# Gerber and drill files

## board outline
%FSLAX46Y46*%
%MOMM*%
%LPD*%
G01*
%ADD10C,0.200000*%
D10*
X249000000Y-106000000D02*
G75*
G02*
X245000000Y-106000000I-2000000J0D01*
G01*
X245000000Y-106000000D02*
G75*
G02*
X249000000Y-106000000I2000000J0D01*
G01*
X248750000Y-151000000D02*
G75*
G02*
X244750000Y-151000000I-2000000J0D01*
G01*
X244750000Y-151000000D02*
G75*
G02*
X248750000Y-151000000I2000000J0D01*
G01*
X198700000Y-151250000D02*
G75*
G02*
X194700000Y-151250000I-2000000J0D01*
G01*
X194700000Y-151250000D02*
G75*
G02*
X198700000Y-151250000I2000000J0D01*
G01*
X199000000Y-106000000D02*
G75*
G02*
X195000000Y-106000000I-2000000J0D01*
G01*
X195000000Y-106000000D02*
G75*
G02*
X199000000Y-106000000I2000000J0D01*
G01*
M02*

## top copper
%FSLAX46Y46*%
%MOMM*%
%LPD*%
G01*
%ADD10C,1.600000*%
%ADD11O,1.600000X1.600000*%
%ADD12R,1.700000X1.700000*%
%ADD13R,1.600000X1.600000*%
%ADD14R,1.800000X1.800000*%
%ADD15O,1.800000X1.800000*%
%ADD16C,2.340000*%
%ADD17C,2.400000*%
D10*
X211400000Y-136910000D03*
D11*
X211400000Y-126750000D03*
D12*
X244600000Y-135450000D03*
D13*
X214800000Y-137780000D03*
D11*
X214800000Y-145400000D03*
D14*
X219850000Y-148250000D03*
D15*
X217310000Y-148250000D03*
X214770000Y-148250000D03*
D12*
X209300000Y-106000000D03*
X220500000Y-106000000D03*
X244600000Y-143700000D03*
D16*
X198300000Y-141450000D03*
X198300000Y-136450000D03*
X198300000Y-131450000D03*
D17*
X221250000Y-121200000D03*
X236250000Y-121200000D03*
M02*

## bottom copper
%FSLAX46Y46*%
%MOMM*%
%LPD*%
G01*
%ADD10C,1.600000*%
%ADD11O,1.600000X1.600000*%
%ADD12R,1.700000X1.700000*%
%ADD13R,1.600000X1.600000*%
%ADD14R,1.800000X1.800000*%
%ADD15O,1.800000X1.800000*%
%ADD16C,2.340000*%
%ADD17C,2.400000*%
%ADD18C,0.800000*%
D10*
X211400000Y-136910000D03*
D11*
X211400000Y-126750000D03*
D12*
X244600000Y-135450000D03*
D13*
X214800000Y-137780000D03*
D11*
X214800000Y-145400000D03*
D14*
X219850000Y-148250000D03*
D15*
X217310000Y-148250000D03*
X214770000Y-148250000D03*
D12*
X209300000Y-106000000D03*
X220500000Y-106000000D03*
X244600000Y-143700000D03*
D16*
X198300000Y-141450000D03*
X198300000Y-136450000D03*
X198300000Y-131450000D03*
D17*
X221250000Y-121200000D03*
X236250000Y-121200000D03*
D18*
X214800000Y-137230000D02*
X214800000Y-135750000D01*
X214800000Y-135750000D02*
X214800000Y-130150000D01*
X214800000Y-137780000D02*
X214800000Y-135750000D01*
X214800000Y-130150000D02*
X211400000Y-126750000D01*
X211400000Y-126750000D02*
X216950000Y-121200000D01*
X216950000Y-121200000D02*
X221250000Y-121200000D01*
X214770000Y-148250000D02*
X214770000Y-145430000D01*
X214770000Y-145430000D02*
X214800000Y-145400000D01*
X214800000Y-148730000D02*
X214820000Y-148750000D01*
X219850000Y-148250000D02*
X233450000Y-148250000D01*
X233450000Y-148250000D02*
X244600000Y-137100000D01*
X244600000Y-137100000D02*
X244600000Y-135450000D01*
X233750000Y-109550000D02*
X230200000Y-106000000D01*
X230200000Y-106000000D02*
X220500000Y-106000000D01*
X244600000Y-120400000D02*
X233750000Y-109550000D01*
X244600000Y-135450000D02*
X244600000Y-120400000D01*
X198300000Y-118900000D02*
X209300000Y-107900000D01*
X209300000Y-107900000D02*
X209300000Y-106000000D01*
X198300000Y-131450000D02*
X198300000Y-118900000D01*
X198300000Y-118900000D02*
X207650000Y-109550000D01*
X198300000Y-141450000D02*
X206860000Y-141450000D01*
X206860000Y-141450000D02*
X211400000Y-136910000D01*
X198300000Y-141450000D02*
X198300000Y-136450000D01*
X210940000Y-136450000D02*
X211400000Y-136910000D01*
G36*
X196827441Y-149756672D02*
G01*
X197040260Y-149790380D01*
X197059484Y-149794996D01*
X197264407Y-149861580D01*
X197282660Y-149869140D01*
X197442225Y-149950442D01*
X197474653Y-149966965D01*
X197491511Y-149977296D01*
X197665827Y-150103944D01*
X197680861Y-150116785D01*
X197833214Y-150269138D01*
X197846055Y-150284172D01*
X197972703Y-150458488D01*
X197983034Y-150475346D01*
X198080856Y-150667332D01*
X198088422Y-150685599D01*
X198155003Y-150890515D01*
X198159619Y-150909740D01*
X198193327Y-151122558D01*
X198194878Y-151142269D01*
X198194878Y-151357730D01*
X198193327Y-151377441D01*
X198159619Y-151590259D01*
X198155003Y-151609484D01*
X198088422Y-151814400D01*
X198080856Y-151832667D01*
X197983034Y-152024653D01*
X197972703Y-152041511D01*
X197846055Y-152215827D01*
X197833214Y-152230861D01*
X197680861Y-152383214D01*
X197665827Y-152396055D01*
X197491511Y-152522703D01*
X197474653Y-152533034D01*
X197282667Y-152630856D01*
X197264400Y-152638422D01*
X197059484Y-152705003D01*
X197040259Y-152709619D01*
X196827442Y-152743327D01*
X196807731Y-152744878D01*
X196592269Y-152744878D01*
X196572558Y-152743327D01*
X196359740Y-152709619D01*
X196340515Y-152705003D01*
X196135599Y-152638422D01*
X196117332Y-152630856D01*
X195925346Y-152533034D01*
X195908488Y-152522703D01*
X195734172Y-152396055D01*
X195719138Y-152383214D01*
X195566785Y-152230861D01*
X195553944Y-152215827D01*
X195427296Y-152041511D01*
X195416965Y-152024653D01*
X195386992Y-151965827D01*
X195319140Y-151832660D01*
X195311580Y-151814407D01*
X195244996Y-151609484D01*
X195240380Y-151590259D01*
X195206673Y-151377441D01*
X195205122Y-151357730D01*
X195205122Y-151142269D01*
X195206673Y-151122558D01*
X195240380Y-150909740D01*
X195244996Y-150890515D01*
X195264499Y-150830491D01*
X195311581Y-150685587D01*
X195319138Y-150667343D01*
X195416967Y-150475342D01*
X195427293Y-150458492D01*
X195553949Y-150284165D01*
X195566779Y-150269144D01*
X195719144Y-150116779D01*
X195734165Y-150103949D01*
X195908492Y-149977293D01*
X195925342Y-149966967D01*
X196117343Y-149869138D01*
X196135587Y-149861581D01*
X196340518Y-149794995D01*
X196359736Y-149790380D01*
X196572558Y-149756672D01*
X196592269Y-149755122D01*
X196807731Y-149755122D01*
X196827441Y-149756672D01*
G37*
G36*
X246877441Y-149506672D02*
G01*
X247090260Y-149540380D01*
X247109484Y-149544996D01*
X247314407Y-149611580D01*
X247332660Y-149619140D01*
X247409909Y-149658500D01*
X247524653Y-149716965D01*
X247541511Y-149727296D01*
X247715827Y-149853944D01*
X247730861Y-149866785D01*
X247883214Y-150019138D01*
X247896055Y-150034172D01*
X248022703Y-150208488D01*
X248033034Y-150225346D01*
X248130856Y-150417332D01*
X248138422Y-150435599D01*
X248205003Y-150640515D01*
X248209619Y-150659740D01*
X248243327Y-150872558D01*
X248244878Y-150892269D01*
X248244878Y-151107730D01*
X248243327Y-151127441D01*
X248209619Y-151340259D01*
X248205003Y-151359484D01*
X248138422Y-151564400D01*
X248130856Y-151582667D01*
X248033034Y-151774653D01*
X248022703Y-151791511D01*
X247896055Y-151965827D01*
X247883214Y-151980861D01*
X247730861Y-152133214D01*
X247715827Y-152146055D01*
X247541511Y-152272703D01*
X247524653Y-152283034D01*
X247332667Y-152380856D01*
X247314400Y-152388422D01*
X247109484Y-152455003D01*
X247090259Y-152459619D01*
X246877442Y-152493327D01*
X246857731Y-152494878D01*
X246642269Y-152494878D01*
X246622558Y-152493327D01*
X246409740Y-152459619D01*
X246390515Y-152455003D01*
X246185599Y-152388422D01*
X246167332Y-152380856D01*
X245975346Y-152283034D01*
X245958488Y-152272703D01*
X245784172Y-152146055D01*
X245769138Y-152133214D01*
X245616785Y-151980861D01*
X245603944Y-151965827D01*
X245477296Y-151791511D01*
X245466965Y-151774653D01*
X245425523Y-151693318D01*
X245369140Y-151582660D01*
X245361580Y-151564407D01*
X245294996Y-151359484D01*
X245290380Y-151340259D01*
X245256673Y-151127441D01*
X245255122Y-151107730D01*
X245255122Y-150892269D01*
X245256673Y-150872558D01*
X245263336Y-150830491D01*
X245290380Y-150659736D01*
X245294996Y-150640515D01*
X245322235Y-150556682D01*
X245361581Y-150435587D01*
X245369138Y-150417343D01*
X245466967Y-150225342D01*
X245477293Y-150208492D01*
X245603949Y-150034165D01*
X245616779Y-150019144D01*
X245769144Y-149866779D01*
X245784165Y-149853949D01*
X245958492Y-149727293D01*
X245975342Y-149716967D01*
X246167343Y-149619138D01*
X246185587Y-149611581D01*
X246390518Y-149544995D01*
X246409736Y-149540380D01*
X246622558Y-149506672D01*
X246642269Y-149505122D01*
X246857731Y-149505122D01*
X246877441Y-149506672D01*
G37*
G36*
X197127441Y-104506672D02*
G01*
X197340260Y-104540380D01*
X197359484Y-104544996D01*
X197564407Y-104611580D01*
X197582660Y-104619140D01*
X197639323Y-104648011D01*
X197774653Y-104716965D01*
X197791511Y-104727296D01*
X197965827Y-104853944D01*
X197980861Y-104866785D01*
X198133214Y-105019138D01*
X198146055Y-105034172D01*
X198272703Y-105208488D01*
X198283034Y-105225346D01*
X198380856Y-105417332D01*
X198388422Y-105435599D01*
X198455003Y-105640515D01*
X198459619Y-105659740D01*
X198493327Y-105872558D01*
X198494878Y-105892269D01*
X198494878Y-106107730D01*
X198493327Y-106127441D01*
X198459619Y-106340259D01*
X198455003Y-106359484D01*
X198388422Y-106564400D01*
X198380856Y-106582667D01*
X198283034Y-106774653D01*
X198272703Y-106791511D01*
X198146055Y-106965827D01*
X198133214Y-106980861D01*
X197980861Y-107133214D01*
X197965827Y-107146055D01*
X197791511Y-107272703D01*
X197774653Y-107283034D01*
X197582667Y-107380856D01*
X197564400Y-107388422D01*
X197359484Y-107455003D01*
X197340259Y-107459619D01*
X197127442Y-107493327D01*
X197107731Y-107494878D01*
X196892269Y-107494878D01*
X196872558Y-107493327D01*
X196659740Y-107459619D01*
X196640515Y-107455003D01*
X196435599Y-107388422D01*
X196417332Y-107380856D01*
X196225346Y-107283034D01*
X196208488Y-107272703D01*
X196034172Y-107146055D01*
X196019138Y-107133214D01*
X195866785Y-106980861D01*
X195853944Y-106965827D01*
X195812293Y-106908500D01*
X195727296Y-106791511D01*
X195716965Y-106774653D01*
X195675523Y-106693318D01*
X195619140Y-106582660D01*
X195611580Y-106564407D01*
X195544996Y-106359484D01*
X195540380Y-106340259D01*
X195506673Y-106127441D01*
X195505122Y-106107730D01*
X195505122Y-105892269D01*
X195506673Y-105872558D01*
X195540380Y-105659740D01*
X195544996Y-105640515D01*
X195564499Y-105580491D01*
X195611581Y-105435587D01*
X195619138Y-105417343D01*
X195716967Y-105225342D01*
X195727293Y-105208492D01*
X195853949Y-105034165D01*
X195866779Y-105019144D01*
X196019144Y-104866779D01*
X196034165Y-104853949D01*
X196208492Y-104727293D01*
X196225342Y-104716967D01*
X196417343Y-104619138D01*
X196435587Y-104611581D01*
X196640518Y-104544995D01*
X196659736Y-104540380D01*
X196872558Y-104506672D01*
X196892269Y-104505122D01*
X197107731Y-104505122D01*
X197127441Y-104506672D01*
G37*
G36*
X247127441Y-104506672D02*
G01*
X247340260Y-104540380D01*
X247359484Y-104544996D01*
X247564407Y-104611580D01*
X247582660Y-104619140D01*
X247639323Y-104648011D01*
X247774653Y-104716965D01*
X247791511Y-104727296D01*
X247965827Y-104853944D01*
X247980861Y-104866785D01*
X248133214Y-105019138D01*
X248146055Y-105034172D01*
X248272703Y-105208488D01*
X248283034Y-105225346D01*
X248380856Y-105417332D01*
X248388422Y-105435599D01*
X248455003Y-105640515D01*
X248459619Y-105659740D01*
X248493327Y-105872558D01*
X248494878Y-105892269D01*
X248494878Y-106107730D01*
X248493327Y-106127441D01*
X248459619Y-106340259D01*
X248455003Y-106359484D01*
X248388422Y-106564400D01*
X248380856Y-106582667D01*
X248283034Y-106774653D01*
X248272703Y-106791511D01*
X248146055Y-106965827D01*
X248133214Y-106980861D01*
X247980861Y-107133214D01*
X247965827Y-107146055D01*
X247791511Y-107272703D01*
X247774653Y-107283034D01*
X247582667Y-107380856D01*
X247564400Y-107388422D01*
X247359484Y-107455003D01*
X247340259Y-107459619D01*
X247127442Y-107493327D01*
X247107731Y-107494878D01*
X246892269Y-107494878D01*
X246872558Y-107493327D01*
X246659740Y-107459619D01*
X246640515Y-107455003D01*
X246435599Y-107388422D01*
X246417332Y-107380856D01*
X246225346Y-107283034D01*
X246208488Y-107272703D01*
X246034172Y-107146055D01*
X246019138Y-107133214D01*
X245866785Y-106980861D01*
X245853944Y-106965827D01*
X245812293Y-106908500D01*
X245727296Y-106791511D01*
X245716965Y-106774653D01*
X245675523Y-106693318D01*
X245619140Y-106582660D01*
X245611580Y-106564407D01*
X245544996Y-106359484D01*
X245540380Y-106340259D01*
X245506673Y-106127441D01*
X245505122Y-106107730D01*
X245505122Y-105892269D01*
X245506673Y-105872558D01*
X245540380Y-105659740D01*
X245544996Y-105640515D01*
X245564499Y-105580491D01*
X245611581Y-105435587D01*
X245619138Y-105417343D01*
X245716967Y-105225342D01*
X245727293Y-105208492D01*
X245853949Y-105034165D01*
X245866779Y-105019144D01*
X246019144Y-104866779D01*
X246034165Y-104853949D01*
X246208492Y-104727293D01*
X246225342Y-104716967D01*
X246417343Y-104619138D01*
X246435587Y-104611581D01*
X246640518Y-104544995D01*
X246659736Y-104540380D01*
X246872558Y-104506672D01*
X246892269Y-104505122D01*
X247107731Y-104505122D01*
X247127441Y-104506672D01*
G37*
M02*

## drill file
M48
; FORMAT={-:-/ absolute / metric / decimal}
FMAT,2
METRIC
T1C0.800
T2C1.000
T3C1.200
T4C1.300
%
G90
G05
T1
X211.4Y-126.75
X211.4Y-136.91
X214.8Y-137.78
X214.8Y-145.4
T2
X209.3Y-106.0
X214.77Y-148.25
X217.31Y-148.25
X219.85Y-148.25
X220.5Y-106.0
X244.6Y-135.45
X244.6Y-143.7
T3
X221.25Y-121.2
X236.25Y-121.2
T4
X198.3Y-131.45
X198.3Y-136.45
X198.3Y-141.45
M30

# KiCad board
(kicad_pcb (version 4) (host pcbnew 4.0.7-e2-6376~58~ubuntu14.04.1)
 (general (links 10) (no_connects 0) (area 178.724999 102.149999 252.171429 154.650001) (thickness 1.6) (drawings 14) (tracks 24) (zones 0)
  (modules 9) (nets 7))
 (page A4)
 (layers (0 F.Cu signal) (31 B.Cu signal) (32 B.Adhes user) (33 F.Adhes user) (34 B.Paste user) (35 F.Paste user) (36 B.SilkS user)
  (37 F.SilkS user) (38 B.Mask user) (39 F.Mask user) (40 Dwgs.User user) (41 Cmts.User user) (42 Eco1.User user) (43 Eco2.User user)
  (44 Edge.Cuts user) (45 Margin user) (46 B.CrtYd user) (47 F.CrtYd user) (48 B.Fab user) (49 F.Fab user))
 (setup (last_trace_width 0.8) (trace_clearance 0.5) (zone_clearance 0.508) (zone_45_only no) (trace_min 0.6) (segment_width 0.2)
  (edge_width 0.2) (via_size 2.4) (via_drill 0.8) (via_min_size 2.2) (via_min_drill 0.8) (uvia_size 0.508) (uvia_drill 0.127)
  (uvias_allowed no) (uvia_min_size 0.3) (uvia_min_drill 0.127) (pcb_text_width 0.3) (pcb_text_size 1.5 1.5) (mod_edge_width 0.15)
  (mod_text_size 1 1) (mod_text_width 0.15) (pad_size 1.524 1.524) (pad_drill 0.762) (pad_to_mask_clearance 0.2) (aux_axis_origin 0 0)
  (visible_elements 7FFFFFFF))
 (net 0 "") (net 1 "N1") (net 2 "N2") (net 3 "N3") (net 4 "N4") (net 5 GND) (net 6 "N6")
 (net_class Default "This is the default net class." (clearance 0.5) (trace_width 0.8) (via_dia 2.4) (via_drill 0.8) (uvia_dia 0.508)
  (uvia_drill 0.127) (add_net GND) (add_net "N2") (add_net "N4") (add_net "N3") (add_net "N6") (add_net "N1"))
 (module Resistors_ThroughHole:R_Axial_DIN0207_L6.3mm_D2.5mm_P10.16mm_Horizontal (layer F.Cu) (at 211.4 136.91 90)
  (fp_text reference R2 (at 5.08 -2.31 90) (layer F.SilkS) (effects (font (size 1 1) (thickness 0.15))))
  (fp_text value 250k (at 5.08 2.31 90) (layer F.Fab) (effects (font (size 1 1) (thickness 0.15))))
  (pad 1 thru_hole circle (at 0 0 90) (size 1.6 1.6) (drill 0.8) (layers *.Cu *.Mask) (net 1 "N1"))
  (pad 2 thru_hole oval (at 10.16 0 90) (size 1.6 1.6) (drill 0.8) (layers *.Cu *.Mask) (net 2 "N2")))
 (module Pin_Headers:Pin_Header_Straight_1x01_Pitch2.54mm (layer F.Cu) (at 244.6 135.45)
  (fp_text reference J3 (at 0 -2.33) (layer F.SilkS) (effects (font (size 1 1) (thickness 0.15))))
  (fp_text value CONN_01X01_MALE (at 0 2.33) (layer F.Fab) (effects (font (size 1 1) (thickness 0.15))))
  (pad 1 thru_hole rect (at 0 0) (size 1.7 1.7) (drill 1) (layers *.Cu *.Mask) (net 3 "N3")))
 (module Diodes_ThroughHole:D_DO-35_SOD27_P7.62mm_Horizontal (layer F.Cu) (at 214.8 137.78 270)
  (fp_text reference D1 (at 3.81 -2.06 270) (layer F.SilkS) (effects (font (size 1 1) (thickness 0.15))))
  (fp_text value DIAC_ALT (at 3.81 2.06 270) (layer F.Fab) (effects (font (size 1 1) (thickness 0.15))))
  (pad 1 thru_hole rect (at 0 0 270) (size 1.6 1.6) (drill 0.8) (layers *.Cu *.Mask) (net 2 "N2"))
  (pad 2 thru_hole oval (at 7.62 0 270) (size 1.6 1.6) (drill 0.8) (layers *.Cu *.Mask) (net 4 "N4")))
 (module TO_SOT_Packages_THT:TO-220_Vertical (layer F.Cu) (at 219.85 148.25 180)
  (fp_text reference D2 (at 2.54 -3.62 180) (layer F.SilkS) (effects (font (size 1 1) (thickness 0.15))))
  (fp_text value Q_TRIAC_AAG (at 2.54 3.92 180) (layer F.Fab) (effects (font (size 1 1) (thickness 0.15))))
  (pad 1 thru_hole rect (at 0 0 180) (size 1.8 1.8) (drill 1) (layers *.Cu *.Mask) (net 3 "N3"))
  (pad 2 thru_hole oval (at 2.54 0 180) (size 1.8 1.8) (drill 1) (layers *.Cu *.Mask) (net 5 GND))
  (pad 3 thru_hole oval (at 5.08 0 180) (size 1.8 1.8) (drill 1) (layers *.Cu *.Mask) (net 4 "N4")))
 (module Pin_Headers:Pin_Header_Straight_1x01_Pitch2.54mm (layer F.Cu) (at 209.3 106)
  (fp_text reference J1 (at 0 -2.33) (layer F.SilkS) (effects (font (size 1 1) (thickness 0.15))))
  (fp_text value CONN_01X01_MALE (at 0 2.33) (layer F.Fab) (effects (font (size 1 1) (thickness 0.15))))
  (pad 1 thru_hole rect (at 0 0) (size 1.7 1.7) (drill 1) (layers *.Cu *.Mask) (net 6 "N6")))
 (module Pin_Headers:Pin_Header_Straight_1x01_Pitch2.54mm (layer F.Cu) (at 220.5 106)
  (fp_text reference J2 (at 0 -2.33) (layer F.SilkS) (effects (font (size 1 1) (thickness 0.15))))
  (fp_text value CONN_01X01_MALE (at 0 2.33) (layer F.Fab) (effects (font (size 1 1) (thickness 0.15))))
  (pad 1 thru_hole rect (at 0 0) (size 1.7 1.7) (drill 1) (layers *.Cu *.Mask) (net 3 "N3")))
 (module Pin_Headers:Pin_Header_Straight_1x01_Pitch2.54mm (layer F.Cu) (at 244.6 143.7)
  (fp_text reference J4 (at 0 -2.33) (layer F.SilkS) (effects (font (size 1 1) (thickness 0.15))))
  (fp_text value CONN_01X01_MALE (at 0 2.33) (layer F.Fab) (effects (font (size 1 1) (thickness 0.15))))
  (pad 1 thru_hole rect (at 0 0) (size 1.7 1.7) (drill 1) (layers *.Cu *.Mask) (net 5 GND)))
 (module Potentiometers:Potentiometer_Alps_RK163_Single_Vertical (layer F.Cu) (at 198.3 131.45 180)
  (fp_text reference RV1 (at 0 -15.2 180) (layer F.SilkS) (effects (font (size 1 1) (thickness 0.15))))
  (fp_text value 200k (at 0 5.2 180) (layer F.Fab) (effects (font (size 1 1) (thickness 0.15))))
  (pad 3 thru_hole circle (at 0 -10 180) (size 2.34 2.34) (drill 1.3) (layers *.Cu *.Mask) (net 1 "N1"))
  (pad 2 thru_hole circle (at 0 -5 180) (size 2.34 2.34) (drill 1.3) (layers *.Cu *.Mask) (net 1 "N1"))
  (pad 1 thru_hole circle (at 0 0 180) (size 2.34 2.34) (drill 1.3) (layers *.Cu *.Mask) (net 6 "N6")))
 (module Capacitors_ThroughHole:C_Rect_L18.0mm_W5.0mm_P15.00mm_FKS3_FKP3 (layer F.Cu) (at 221.25 121.2)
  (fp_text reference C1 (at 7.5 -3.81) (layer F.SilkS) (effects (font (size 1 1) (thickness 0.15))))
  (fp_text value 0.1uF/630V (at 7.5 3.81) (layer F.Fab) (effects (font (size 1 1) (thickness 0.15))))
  (pad 1 thru_hole circle (at 0 0) (size 2.4 2.4) (drill 1.2) (layers *.Cu *.Mask) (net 2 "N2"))
  (pad 2 thru_hole circle (at 15 0) (size 2.4 2.4) (drill 1.2) (layers *.Cu *.Mask) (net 5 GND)))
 (gr_circle (center 247 106) (end 249 106) (layer Edge.Cuts) (width 0.2))
 (gr_circle (center 246.75 151) (end 248.75 151) (layer Edge.Cuts) (width 0.2))
 (gr_circle (center 196.7 151.25) (end 198.7 151.25) (layer Edge.Cuts) (width 0.2))
 (gr_circle (center 197 106) (end 199 106) (layer Edge.Cuts) (width 0.2))
 (segment (start 214.8 137.23) (end 214.8 135.75) (width 0.8) (layer B.Cu) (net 2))
 (segment (start 214.8 135.75) (end 214.8 130.15) (width 0.8) (layer B.Cu) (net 2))
 (segment (start 214.8 137.78) (end 214.8 135.75) (width 0.8) (layer B.Cu) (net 2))
 (segment (start 214.8 130.15) (end 211.4 126.75) (width 0.8) (layer B.Cu) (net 2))
 (segment (start 211.4 126.75) (end 216.95 121.2) (width 0.8) (layer B.Cu) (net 2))
 (segment (start 216.95 121.2) (end 221.25 121.2) (width 0.8) (layer B.Cu) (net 2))
 (segment (start 214.77 148.25) (end 214.77 145.43) (width 0.8) (layer B.Cu) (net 4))
 (segment (start 214.77 145.43) (end 214.8 145.4) (width 0.8) (layer B.Cu) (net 4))
 (segment (start 214.8 148.73) (end 214.82 148.75) (width 0.8) (layer B.Cu) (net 4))
 (segment (start 219.85 148.25) (end 233.45 148.25) (width 0.8) (layer B.Cu) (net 3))
 (segment (start 233.45 148.25) (end 244.6 137.1) (width 0.8) (layer B.Cu) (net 3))
 (segment (start 244.6 137.1) (end 244.6 135.45) (width 0.8) (layer B.Cu) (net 3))
 (segment (start 233.75 109.55) (end 230.2 106) (width 0.8) (layer B.Cu) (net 3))
 (segment (start 230.2 106) (end 220.5 106) (width 0.8) (layer B.Cu) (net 3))
 (segment (start 244.6 120.4) (end 233.75 109.55) (width 0.8) (layer B.Cu) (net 3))
 (segment (start 244.6 135.45) (end 244.6 120.4) (width 0.8) (layer B.Cu) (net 3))
 (segment (start 198.3 118.9) (end 209.3 107.9) (width 0.8) (layer B.Cu) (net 6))
 (segment (start 209.3 107.9) (end 209.3 106) (width 0.8) (layer B.Cu) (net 6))
 (segment (start 198.3 131.45) (end 198.3 118.9) (width 0.8) (layer B.Cu) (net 6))
 (segment (start 198.3 118.9) (end 207.65 109.55) (width 0.8) (layer B.Cu) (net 6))
 (segment (start 198.3 141.45) (end 206.86 141.45) (width 0.8) (layer B.Cu) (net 1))
 (segment (start 206.86 141.45) (end 211.4 136.91) (width 0.8) (layer B.Cu) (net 1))
 (segment (start 198.3 141.45) (end 198.3 136.45) (width 0.8) (layer B.Cu) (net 1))
 (segment (start 210.94 136.45) (end 211.4 136.91) (width 0.8) (layer B.Cu) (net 1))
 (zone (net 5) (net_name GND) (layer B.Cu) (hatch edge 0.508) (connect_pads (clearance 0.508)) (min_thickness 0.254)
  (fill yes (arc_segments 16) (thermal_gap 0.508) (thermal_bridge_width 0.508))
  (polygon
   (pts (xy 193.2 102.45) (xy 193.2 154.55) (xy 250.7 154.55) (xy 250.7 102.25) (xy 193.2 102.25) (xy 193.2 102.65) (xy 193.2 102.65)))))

